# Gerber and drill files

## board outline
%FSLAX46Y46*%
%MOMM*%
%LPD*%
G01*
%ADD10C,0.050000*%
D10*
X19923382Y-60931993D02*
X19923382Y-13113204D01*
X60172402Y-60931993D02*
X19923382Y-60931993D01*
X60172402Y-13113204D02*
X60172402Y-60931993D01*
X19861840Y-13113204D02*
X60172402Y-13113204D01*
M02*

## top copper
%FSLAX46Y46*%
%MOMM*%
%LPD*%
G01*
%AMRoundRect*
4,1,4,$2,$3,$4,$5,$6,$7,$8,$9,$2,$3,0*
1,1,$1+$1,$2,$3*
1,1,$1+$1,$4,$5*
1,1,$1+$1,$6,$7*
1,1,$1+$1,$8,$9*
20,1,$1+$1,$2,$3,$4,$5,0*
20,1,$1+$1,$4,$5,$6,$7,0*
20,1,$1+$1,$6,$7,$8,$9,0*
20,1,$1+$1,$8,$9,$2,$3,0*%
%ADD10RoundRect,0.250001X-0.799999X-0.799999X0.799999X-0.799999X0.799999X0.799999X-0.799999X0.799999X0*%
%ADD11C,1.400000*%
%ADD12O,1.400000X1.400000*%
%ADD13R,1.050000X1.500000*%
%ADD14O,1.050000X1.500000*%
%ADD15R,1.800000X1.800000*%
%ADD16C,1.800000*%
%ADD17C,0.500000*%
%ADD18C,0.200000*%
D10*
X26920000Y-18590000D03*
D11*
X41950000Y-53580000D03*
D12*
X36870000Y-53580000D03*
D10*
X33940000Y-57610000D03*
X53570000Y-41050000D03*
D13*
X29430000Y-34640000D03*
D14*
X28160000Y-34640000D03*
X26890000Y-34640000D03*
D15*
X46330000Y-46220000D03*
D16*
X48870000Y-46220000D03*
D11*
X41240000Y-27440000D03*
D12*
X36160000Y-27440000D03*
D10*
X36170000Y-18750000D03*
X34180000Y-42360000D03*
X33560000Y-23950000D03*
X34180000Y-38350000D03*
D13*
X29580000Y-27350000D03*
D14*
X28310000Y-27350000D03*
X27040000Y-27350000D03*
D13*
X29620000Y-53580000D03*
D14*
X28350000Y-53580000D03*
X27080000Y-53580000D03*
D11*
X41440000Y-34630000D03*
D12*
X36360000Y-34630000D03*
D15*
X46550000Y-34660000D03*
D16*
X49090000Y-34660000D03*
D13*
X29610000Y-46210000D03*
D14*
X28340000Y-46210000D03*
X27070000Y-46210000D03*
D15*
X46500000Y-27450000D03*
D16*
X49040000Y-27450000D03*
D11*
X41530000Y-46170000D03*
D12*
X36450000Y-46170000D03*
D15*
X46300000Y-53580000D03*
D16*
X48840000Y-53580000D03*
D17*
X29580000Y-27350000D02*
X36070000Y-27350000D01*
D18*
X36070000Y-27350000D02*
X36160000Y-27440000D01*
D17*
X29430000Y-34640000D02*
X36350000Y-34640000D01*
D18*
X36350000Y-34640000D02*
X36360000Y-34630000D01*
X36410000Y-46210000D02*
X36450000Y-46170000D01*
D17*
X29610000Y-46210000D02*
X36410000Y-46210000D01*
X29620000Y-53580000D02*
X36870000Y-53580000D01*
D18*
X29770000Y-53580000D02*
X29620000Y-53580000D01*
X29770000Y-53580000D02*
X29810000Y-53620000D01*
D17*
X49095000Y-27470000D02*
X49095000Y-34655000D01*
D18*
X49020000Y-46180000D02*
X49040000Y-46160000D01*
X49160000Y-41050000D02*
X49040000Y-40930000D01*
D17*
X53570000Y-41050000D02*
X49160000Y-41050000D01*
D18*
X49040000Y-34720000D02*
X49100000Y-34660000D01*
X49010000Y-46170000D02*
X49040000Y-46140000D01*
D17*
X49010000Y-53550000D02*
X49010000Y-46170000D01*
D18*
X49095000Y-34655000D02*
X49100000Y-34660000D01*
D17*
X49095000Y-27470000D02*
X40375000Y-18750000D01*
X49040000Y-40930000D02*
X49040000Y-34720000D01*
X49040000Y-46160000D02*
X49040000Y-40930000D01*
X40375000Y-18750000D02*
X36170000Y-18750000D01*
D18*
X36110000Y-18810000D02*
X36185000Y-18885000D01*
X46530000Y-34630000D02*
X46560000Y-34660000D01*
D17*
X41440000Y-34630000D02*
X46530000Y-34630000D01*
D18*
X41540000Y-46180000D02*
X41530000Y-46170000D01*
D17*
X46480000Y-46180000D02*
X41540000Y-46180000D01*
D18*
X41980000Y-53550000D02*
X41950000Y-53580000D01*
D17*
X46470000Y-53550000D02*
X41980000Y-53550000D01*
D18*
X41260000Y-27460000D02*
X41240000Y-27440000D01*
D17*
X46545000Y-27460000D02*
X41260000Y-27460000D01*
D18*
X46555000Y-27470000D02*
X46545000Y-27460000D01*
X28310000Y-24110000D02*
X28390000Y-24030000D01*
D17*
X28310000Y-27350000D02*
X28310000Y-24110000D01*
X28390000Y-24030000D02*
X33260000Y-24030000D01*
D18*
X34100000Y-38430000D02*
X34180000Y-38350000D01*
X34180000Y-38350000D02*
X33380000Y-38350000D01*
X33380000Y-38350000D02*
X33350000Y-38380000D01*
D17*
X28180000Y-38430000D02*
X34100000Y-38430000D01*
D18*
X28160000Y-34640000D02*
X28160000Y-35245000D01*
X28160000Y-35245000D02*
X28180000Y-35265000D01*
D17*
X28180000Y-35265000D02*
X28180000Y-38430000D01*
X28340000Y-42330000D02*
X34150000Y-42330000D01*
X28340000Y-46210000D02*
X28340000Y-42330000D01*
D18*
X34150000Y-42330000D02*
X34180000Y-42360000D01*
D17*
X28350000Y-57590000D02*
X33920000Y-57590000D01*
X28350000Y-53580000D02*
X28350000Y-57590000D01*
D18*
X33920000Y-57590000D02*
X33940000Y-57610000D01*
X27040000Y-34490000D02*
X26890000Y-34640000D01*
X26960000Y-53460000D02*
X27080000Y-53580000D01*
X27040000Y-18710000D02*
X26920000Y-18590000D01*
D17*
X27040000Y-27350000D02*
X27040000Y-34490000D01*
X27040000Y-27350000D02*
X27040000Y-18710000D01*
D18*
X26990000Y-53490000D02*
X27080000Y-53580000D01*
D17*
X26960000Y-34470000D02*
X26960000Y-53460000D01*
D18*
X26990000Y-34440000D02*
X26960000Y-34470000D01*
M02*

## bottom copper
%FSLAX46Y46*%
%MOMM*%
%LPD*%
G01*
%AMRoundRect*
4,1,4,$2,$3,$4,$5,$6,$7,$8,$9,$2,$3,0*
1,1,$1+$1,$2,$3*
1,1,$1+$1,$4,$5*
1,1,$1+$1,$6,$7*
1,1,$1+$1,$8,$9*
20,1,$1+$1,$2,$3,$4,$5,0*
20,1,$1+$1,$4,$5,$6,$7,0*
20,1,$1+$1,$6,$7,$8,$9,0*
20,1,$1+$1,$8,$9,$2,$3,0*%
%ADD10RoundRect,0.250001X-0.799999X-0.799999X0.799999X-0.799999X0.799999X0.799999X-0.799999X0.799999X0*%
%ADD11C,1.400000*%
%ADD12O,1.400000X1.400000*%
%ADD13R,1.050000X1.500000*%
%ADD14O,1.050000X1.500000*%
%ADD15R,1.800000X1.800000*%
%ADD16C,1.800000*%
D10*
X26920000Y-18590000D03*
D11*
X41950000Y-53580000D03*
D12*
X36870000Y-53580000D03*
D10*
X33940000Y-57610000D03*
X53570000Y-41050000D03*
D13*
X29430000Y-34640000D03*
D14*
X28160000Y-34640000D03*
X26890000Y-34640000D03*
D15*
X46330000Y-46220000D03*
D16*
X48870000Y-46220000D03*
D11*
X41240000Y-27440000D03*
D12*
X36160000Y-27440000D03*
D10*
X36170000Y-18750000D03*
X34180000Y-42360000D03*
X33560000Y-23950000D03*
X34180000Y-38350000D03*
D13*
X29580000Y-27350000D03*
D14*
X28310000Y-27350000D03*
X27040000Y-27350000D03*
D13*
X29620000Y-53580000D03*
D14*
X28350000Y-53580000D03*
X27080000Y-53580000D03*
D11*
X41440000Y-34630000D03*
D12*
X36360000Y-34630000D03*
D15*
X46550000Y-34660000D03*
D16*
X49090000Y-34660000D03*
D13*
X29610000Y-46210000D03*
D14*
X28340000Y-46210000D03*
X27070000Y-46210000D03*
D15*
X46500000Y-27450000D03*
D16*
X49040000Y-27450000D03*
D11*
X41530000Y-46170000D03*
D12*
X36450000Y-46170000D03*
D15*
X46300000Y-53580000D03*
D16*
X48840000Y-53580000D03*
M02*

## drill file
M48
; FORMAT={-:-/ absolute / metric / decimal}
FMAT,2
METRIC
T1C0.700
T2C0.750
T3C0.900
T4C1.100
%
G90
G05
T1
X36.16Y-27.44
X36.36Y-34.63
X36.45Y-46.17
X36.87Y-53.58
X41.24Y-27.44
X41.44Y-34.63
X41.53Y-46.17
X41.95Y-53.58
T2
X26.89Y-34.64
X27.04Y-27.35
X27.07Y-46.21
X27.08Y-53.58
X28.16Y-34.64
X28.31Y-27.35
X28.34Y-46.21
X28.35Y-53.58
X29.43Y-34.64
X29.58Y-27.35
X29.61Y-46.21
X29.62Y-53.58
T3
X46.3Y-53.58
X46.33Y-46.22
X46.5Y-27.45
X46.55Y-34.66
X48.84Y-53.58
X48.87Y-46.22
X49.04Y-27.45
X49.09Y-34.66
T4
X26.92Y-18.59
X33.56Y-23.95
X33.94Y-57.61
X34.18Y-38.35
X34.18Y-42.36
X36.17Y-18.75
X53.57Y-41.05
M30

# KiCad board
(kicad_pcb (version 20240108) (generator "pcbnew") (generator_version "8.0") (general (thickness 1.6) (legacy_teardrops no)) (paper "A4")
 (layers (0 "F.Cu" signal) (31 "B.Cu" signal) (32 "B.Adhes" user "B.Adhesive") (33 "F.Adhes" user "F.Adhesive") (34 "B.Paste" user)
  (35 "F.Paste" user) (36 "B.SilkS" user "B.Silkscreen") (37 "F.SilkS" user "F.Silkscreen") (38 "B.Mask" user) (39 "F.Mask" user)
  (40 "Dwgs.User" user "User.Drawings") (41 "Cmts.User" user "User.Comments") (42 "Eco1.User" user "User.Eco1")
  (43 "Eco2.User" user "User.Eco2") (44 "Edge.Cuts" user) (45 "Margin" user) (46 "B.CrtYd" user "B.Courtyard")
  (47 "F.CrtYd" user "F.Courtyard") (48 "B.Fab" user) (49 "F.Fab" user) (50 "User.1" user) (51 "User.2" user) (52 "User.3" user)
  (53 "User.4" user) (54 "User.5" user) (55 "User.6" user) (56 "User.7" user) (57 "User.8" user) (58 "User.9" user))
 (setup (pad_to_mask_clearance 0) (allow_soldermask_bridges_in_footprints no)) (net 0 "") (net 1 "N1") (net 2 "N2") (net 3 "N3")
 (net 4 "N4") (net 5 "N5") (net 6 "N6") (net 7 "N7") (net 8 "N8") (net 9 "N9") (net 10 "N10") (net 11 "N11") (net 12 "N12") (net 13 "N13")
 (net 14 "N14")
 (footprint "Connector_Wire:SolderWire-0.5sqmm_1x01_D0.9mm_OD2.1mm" (layer "F.Cu") (at 26.92 18.59)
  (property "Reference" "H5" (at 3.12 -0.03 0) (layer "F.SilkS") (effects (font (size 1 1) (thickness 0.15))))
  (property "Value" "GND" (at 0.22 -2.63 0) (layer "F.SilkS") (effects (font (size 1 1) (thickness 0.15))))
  (pad "1" thru_hole roundrect (at 0 0) (size 2.1 2.1) (drill 1.1) (layers "*.Cu" "*.Mask") (remove_unused_layers no)
   (roundrect_rratio 0.119048) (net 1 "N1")))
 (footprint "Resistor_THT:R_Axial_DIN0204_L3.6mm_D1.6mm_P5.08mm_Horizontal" (layer "F.Cu") (at 41.95 53.58 180)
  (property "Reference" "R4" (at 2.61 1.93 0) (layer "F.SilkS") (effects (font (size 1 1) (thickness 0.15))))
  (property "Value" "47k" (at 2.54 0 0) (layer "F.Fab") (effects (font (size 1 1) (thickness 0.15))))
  (pad "1" thru_hole circle (at 0 0 180) (size 1.4 1.4) (drill 0.7) (layers "*.Cu" "*.Mask") (remove_unused_layers no) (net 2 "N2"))
  (pad "2" thru_hole oval (at 5.08 0 180) (size 1.4 1.4) (drill 0.7) (layers "*.Cu" "*.Mask") (remove_unused_layers no) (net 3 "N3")))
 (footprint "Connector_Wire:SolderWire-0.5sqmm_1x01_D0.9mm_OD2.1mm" (layer "F.Cu") (at 33.94 57.61)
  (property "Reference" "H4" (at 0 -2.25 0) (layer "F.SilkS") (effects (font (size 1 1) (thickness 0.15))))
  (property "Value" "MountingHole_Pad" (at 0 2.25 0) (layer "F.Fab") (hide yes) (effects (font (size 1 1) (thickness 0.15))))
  (pad "1" thru_hole roundrect (at 0 0) (size 2.1 2.1) (drill 1.1) (layers "*.Cu" "*.Mask") (remove_unused_layers no)
   (roundrect_rratio 0.119048) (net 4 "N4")))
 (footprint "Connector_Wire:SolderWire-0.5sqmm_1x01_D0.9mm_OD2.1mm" (layer "F.Cu") (at 53.57 41.05)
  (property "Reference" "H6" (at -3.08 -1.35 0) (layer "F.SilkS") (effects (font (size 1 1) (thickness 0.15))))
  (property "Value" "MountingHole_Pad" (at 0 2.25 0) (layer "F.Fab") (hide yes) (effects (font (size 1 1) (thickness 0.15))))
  (pad "1" thru_hole roundrect (at 0 0) (size 2.1 2.1) (drill 1.1) (layers "*.Cu" "*.Mask") (remove_unused_layers no)
   (roundrect_rratio 0.119048) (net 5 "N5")))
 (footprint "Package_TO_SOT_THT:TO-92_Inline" (layer "F.Cu") (at 29.43 34.64 180)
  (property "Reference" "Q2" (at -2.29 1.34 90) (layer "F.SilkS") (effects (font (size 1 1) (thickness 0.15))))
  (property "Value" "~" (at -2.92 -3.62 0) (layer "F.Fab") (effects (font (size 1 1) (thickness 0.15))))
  (pad "1" thru_hole rect (at 0 0 180) (size 1.05 1.5) (drill 0.75) (layers "*.Cu" "*.Mask") (remove_unused_layers no) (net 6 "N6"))
  (pad "2" thru_hole oval (at 1.27 0 180) (size 1.05 1.5) (drill 0.75) (layers "*.Cu" "*.Mask") (remove_unused_layers no) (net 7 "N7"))
  (pad "3" thru_hole oval (at 2.54 0 180) (size 1.05 1.5) (drill 0.75) (layers "*.Cu" "*.Mask") (remove_unused_layers no) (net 1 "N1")))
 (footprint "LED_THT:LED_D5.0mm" (layer "F.Cu") (at 46.33 46.22)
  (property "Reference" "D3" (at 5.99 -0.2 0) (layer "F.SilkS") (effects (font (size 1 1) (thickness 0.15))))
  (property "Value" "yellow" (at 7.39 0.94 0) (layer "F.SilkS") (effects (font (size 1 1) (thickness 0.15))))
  (pad "1" thru_hole rect (at 0 0) (size 1.8 1.8) (drill 0.9) (layers "*.Cu" "*.Mask") (remove_unused_layers no) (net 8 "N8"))
  (pad "2" thru_hole circle (at 2.54 0) (size 1.8 1.8) (drill 0.9) (layers "*.Cu" "*.Mask") (remove_unused_layers no) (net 5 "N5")))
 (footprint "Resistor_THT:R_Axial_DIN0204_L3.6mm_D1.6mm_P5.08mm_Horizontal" (layer "F.Cu") (at 41.24 27.44 180)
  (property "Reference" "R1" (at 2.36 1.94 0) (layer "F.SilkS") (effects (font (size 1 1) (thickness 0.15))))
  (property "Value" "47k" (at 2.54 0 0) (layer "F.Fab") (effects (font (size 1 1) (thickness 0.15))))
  (pad "1" thru_hole circle (at 0 0 180) (size 1.4 1.4) (drill 0.7) (layers "*.Cu" "*.Mask") (remove_unused_layers no) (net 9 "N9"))
  (pad "2" thru_hole oval (at 5.08 0 180) (size 1.4 1.4) (drill 0.7) (layers "*.Cu" "*.Mask") (remove_unused_layers no) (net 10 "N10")))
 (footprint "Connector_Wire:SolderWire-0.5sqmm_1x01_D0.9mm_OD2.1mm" (layer "F.Cu") (at 36.17 18.75)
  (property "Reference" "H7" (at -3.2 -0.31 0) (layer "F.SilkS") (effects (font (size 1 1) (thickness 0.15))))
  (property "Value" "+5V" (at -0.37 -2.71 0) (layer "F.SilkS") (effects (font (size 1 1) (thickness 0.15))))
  (pad "1" thru_hole roundrect (at 0 0) (size 2.1 2.1) (drill 1.1) (layers "*.Cu" "*.Mask") (remove_unused_layers no)
   (roundrect_rratio 0.119048) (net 5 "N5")))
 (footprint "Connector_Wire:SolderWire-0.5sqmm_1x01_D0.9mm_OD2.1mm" (layer "F.Cu") (at 34.18 42.36)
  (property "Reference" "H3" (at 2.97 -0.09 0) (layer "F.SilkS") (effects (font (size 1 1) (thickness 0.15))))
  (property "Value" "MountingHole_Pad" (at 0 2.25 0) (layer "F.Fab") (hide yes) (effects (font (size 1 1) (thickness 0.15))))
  (pad "1" thru_hole roundrect (at 0 0) (size 2.1 2.1) (drill 1.1) (layers "*.Cu" "*.Mask") (remove_unused_layers no)
   (roundrect_rratio 0.119048) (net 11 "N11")))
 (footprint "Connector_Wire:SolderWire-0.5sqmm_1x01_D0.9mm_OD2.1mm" (layer "F.Cu") (at 33.56 23.95)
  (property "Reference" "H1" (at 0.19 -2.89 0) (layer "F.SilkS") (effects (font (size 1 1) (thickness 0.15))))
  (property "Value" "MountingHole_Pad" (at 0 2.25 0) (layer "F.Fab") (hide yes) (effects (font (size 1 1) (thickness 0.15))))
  (pad "1" thru_hole roundrect (at 0 0) (size 2.1 2.1) (drill 1.1) (layers "*.Cu" "*.Mask") (remove_unused_layers no)
   (roundrect_rratio 0.119048) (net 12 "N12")))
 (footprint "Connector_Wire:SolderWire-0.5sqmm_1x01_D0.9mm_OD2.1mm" (layer "F.Cu") (at 34.18 38.35)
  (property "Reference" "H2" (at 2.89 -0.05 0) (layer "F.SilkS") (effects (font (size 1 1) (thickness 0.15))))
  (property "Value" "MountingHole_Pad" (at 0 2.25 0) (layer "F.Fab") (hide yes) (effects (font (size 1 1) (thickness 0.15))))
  (pad "1" thru_hole roundrect (at 0 0) (size 2.1 2.1) (drill 1.1) (layers "*.Cu" "*.Mask") (remove_unused_layers no)
   (roundrect_rratio 0.119048) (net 7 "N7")))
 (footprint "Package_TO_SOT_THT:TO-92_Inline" (layer "F.Cu") (at 29.58 27.35 180)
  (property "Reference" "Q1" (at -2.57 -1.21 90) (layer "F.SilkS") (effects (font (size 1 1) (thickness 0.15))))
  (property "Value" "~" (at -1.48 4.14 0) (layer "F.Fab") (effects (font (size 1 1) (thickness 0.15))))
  (pad "1" thru_hole rect (at 0 0 180) (size 1.05 1.5) (drill 0.75) (layers "*.Cu" "*.Mask") (remove_unused_layers no) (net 10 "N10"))
  (pad "2" thru_hole oval (at 1.27 0 180) (size 1.05 1.5) (drill 0.75) (layers "*.Cu" "*.Mask") (remove_unused_layers no) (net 12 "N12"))
  (pad "3" thru_hole oval (at 2.54 0 180) (size 1.05 1.5) (drill 0.75) (layers "*.Cu" "*.Mask") (remove_unused_layers no) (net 1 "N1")))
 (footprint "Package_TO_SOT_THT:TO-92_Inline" (layer "F.Cu") (at 29.62 53.58 180)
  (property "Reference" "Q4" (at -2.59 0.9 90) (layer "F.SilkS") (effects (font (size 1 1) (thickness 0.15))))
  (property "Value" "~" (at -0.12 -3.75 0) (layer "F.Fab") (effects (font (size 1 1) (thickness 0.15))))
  (pad "1" thru_hole rect (at 0 0 180) (size 1.05 1.5) (drill 0.75) (layers "*.Cu" "*.Mask") (remove_unused_layers no) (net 3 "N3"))
  (pad "2" thru_hole oval (at 1.27 0 180) (size 1.05 1.5) (drill 0.75) (layers "*.Cu" "*.Mask") (remove_unused_layers no) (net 4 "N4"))
  (pad "3" thru_hole oval (at 2.54 0 180) (size 1.05 1.5) (drill 0.75) (layers "*.Cu" "*.Mask") (remove_unused_layers no) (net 1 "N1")))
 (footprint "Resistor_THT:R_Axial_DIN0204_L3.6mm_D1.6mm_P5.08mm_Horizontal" (layer "F.Cu") (at 41.44 34.63 180)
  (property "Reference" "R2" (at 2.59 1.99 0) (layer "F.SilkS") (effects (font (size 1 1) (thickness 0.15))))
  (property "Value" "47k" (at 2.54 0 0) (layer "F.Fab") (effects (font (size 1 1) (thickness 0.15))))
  (pad "1" thru_hole circle (at 0 0 180) (size 1.4 1.4) (drill 0.7) (layers "*.Cu" "*.Mask") (remove_unused_layers no) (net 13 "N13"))
  (pad "2" thru_hole oval (at 5.08 0 180) (size 1.4 1.4) (drill 0.7) (layers "*.Cu" "*.Mask") (remove_unused_layers no) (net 6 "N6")))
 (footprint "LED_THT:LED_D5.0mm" (layer "F.Cu") (at 46.55 34.66)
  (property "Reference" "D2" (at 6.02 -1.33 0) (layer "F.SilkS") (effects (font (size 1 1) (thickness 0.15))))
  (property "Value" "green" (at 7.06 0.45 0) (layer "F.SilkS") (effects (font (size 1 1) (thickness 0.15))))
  (pad "1" thru_hole rect (at 0 0) (size 1.8 1.8) (drill 0.9) (layers "*.Cu" "*.Mask") (remove_unused_layers no) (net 13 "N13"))
  (pad "2" thru_hole circle (at 2.54 0) (size 1.8 1.8) (drill 0.9) (layers "*.Cu" "*.Mask") (remove_unused_layers no) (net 5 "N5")))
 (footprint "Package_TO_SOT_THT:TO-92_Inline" (layer "F.Cu") (at 29.61 46.21 180)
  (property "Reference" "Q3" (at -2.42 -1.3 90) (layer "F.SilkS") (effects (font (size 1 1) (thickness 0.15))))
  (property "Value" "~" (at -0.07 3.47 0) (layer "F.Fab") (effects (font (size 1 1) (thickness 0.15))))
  (pad "1" thru_hole rect (at 0 0 180) (size 1.05 1.5) (drill 0.75) (layers "*.Cu" "*.Mask") (remove_unused_layers no) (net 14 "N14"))
  (pad "2" thru_hole oval (at 1.27 0 180) (size 1.05 1.5) (drill 0.75) (layers "*.Cu" "*.Mask") (remove_unused_layers no) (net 11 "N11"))
  (pad "3" thru_hole oval (at 2.54 0 180) (size 1.05 1.5) (drill 0.75) (layers "*.Cu" "*.Mask") (remove_unused_layers no) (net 1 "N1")))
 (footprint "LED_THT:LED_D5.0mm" (layer "F.Cu") (at 46.5 27.45)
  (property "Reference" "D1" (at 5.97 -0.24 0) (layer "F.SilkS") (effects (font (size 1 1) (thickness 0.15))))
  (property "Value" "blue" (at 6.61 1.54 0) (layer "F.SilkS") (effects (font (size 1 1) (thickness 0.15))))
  (pad "1" thru_hole rect (at 0 0) (size 1.8 1.8) (drill 0.9) (layers "*.Cu" "*.Mask") (remove_unused_layers no) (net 9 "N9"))
  (pad "2" thru_hole circle (at 2.54 0) (size 1.8 1.8) (drill 0.9) (layers "*.Cu" "*.Mask") (remove_unused_layers no) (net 5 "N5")))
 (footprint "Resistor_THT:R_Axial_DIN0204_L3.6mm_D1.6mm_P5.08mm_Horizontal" (layer "F.Cu") (at 41.53 46.17 180)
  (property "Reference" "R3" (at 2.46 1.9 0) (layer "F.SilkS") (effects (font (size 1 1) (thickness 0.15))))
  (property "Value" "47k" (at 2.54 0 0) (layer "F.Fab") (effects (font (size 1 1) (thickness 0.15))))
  (pad "1" thru_hole circle (at 0 0 180) (size 1.4 1.4) (drill 0.7) (layers "*.Cu" "*.Mask") (remove_unused_layers no) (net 8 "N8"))
  (pad "2" thru_hole oval (at 5.08 0 180) (size 1.4 1.4) (drill 0.7) (layers "*.Cu" "*.Mask") (remove_unused_layers no) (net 14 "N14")))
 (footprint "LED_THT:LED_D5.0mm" (layer "F.Cu") (at 46.3 53.58)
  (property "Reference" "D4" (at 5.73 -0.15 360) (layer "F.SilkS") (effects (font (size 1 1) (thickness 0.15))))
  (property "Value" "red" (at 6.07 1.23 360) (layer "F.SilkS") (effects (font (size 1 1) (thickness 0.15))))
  (pad "1" thru_hole rect (at 0 0) (size 1.8 1.8) (drill 0.9) (layers "*.Cu" "*.Mask") (remove_unused_layers no) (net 2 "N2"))
  (pad "2" thru_hole circle (at 2.54 0) (size 1.8 1.8) (drill 0.9) (layers "*.Cu" "*.Mask") (remove_unused_layers no) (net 5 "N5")))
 (gr_line (start 19.923382 60.931993) (end 19.923382 13.113204) (stroke (width 0.05) (type default)) (layer "Edge.Cuts"))
 (gr_line (start 60.172402 60.931993) (end 19.923382 60.931993) (stroke (width 0.05) (type default)) (layer "Edge.Cuts"))
 (gr_line (start 60.172402 13.113204) (end 60.172402 60.931993) (stroke (width 0.05) (type default)) (layer "Edge.Cuts"))
 (gr_line (start 19.86184 13.113204) (end 60.172402 13.113204) (stroke (width 0.05) (type default)) (layer "Edge.Cuts"))
 (segment (start 29.58 27.35) (end 36.07 27.35) (width 0.5) (layer "F.Cu") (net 10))
 (segment (start 36.07 27.35) (end 36.16 27.44) (width 0.2) (layer "F.Cu") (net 10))
 (segment (start 29.43 34.64) (end 36.35 34.64) (width 0.5) (layer "F.Cu") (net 6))
 (segment (start 36.35 34.64) (end 36.36 34.63) (width 0.2) (layer "F.Cu") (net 6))
 (segment (start 36.41 46.21) (end 36.45 46.17) (width 0.2) (layer "F.Cu") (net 14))
 (segment (start 29.61 46.21) (end 36.41 46.21) (width 0.5) (layer "F.Cu") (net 14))
 (segment (start 29.62 53.58) (end 36.87 53.58) (width 0.5) (layer "F.Cu") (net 3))
 (segment (start 29.77 53.58) (end 29.62 53.58) (width 0.2) (layer "F.Cu") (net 3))
 (segment (start 29.77 53.58) (end 29.81 53.62) (width 0.2) (layer "F.Cu") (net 3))
 (segment (start 49.095 27.47) (end 49.095 34.655) (width 0.5) (layer "F.Cu") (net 5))
 (segment (start 49.02 46.18) (end 49.04 46.16) (width 0.2) (layer "F.Cu") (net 5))
 (segment (start 49.16 41.05) (end 49.04 40.93) (width 0.2) (layer "F.Cu") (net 5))
 (segment (start 53.57 41.05) (end 49.16 41.05) (width 0.5) (layer "F.Cu") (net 5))
 (segment (start 49.04 34.72) (end 49.1 34.66) (width 0.2) (layer "F.Cu") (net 5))
 (segment (start 49.01 46.17) (end 49.04 46.14) (width 0.2) (layer "F.Cu") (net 5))
 (segment (start 49.01 53.55) (end 49.01 46.17) (width 0.5) (layer "F.Cu") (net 5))
 (segment (start 49.095 34.655) (end 49.1 34.66) (width 0.2) (layer "F.Cu") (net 5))
 (segment (start 49.095 27.47) (end 40.375 18.75) (width 0.5) (layer "F.Cu") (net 5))
 (segment (start 49.04 40.93) (end 49.04 34.72) (width 0.5) (layer "F.Cu") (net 5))
 (segment (start 49.04 46.16) (end 49.04 40.93) (width 0.5) (layer "F.Cu") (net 5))
 (segment (start 40.375 18.75) (end 36.17 18.75) (width 0.5) (layer "F.Cu") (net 5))
 (segment (start 36.11 18.81) (end 36.185 18.885) (width 0.2) (layer "F.Cu") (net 5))
 (segment (start 46.53 34.63) (end 46.56 34.66) (width 0.2) (layer "F.Cu") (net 13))
 (segment (start 41.44 34.63) (end 46.53 34.63) (width 0.5) (layer "F.Cu") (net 13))
 (segment (start 41.54 46.18) (end 41.53 46.17) (width 0.2) (layer "F.Cu") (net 8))
 (segment (start 46.48 46.18) (end 41.54 46.18) (width 0.5) (layer "F.Cu") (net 8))
 (segment (start 41.98 53.55) (end 41.95 53.58) (width 0.2) (layer "F.Cu") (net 2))
 (segment (start 46.47 53.55) (end 41.98 53.55) (width 0.5) (layer "F.Cu") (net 2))
 (segment (start 41.26 27.46) (end 41.24 27.44) (width 0.2) (layer "F.Cu") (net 9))
 (segment (start 46.545 27.46) (end 41.26 27.46) (width 0.5) (layer "F.Cu") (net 9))
 (segment (start 46.555 27.47) (end 46.545 27.46) (width 0.2) (layer "F.Cu") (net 9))
 (segment (start 28.31 24.11) (end 28.39 24.03) (width 0.2) (layer "F.Cu") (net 12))
 (segment (start 28.31 27.35) (end 28.31 24.11) (width 0.5) (layer "F.Cu") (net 12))
 (segment (start 28.39 24.03) (end 33.26 24.03) (width 0.5) (layer "F.Cu") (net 12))
 (segment (start 34.1 38.43) (end 34.18 38.35) (width 0.2) (layer "F.Cu") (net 7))
 (segment (start 34.18 38.35) (end 33.38 38.35) (width 0.2) (layer "F.Cu") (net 7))
 (segment (start 33.38 38.35) (end 33.35 38.38) (width 0.2) (layer "F.Cu") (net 7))
 (segment (start 28.18 38.43) (end 34.1 38.43) (width 0.5) (layer "F.Cu") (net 7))
 (segment (start 28.16 34.64) (end 28.16 35.245) (width 0.2) (layer "F.Cu") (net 7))
 (segment (start 28.16 35.245) (end 28.18 35.265) (width 0.2) (layer "F.Cu") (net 7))
 (segment (start 28.18 35.265) (end 28.18 38.43) (width 0.5) (layer "F.Cu") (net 7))
 (segment (start 28.34 42.33) (end 34.15 42.33) (width 0.5) (layer "F.Cu") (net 11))
 (segment (start 28.34 46.21) (end 28.34 42.33) (width 0.5) (layer "F.Cu") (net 11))
 (segment (start 34.15 42.33) (end 34.18 42.36) (width 0.2) (layer "F.Cu") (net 11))
 (segment (start 28.35 57.59) (end 33.92 57.59) (width 0.5) (layer "F.Cu") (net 4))
 (segment (start 28.35 53.58) (end 28.35 57.59) (width 0.5) (layer "F.Cu") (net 4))
 (segment (start 33.92 57.59) (end 33.94 57.61) (width 0.2) (layer "F.Cu") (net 4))
 (segment (start 27.04 34.49) (end 26.89 34.64) (width 0.2) (layer "F.Cu") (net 1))
 (segment (start 26.96 53.46) (end 27.08 53.58) (width 0.2) (layer "F.Cu") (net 1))
 (segment (start 27.04 18.71) (end 26.92 18.59) (width 0.2) (layer "F.Cu") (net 1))
 (segment (start 27.04 27.35) (end 27.04 34.49) (width 0.5) (layer "F.Cu") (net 1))
 (segment (start 27.04 27.35) (end 27.04 18.71) (width 0.5) (layer "F.Cu") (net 1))
 (segment (start 26.99 53.49) (end 27.08 53.58) (width 0.2) (layer "F.Cu") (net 1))
 (segment (start 26.96 34.47) (end 26.96 53.46) (width 0.5) (layer "F.Cu") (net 1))
 (segment (start 26.99 34.44) (end 26.96 34.47) (width 0.2) (layer "F.Cu") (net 1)))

